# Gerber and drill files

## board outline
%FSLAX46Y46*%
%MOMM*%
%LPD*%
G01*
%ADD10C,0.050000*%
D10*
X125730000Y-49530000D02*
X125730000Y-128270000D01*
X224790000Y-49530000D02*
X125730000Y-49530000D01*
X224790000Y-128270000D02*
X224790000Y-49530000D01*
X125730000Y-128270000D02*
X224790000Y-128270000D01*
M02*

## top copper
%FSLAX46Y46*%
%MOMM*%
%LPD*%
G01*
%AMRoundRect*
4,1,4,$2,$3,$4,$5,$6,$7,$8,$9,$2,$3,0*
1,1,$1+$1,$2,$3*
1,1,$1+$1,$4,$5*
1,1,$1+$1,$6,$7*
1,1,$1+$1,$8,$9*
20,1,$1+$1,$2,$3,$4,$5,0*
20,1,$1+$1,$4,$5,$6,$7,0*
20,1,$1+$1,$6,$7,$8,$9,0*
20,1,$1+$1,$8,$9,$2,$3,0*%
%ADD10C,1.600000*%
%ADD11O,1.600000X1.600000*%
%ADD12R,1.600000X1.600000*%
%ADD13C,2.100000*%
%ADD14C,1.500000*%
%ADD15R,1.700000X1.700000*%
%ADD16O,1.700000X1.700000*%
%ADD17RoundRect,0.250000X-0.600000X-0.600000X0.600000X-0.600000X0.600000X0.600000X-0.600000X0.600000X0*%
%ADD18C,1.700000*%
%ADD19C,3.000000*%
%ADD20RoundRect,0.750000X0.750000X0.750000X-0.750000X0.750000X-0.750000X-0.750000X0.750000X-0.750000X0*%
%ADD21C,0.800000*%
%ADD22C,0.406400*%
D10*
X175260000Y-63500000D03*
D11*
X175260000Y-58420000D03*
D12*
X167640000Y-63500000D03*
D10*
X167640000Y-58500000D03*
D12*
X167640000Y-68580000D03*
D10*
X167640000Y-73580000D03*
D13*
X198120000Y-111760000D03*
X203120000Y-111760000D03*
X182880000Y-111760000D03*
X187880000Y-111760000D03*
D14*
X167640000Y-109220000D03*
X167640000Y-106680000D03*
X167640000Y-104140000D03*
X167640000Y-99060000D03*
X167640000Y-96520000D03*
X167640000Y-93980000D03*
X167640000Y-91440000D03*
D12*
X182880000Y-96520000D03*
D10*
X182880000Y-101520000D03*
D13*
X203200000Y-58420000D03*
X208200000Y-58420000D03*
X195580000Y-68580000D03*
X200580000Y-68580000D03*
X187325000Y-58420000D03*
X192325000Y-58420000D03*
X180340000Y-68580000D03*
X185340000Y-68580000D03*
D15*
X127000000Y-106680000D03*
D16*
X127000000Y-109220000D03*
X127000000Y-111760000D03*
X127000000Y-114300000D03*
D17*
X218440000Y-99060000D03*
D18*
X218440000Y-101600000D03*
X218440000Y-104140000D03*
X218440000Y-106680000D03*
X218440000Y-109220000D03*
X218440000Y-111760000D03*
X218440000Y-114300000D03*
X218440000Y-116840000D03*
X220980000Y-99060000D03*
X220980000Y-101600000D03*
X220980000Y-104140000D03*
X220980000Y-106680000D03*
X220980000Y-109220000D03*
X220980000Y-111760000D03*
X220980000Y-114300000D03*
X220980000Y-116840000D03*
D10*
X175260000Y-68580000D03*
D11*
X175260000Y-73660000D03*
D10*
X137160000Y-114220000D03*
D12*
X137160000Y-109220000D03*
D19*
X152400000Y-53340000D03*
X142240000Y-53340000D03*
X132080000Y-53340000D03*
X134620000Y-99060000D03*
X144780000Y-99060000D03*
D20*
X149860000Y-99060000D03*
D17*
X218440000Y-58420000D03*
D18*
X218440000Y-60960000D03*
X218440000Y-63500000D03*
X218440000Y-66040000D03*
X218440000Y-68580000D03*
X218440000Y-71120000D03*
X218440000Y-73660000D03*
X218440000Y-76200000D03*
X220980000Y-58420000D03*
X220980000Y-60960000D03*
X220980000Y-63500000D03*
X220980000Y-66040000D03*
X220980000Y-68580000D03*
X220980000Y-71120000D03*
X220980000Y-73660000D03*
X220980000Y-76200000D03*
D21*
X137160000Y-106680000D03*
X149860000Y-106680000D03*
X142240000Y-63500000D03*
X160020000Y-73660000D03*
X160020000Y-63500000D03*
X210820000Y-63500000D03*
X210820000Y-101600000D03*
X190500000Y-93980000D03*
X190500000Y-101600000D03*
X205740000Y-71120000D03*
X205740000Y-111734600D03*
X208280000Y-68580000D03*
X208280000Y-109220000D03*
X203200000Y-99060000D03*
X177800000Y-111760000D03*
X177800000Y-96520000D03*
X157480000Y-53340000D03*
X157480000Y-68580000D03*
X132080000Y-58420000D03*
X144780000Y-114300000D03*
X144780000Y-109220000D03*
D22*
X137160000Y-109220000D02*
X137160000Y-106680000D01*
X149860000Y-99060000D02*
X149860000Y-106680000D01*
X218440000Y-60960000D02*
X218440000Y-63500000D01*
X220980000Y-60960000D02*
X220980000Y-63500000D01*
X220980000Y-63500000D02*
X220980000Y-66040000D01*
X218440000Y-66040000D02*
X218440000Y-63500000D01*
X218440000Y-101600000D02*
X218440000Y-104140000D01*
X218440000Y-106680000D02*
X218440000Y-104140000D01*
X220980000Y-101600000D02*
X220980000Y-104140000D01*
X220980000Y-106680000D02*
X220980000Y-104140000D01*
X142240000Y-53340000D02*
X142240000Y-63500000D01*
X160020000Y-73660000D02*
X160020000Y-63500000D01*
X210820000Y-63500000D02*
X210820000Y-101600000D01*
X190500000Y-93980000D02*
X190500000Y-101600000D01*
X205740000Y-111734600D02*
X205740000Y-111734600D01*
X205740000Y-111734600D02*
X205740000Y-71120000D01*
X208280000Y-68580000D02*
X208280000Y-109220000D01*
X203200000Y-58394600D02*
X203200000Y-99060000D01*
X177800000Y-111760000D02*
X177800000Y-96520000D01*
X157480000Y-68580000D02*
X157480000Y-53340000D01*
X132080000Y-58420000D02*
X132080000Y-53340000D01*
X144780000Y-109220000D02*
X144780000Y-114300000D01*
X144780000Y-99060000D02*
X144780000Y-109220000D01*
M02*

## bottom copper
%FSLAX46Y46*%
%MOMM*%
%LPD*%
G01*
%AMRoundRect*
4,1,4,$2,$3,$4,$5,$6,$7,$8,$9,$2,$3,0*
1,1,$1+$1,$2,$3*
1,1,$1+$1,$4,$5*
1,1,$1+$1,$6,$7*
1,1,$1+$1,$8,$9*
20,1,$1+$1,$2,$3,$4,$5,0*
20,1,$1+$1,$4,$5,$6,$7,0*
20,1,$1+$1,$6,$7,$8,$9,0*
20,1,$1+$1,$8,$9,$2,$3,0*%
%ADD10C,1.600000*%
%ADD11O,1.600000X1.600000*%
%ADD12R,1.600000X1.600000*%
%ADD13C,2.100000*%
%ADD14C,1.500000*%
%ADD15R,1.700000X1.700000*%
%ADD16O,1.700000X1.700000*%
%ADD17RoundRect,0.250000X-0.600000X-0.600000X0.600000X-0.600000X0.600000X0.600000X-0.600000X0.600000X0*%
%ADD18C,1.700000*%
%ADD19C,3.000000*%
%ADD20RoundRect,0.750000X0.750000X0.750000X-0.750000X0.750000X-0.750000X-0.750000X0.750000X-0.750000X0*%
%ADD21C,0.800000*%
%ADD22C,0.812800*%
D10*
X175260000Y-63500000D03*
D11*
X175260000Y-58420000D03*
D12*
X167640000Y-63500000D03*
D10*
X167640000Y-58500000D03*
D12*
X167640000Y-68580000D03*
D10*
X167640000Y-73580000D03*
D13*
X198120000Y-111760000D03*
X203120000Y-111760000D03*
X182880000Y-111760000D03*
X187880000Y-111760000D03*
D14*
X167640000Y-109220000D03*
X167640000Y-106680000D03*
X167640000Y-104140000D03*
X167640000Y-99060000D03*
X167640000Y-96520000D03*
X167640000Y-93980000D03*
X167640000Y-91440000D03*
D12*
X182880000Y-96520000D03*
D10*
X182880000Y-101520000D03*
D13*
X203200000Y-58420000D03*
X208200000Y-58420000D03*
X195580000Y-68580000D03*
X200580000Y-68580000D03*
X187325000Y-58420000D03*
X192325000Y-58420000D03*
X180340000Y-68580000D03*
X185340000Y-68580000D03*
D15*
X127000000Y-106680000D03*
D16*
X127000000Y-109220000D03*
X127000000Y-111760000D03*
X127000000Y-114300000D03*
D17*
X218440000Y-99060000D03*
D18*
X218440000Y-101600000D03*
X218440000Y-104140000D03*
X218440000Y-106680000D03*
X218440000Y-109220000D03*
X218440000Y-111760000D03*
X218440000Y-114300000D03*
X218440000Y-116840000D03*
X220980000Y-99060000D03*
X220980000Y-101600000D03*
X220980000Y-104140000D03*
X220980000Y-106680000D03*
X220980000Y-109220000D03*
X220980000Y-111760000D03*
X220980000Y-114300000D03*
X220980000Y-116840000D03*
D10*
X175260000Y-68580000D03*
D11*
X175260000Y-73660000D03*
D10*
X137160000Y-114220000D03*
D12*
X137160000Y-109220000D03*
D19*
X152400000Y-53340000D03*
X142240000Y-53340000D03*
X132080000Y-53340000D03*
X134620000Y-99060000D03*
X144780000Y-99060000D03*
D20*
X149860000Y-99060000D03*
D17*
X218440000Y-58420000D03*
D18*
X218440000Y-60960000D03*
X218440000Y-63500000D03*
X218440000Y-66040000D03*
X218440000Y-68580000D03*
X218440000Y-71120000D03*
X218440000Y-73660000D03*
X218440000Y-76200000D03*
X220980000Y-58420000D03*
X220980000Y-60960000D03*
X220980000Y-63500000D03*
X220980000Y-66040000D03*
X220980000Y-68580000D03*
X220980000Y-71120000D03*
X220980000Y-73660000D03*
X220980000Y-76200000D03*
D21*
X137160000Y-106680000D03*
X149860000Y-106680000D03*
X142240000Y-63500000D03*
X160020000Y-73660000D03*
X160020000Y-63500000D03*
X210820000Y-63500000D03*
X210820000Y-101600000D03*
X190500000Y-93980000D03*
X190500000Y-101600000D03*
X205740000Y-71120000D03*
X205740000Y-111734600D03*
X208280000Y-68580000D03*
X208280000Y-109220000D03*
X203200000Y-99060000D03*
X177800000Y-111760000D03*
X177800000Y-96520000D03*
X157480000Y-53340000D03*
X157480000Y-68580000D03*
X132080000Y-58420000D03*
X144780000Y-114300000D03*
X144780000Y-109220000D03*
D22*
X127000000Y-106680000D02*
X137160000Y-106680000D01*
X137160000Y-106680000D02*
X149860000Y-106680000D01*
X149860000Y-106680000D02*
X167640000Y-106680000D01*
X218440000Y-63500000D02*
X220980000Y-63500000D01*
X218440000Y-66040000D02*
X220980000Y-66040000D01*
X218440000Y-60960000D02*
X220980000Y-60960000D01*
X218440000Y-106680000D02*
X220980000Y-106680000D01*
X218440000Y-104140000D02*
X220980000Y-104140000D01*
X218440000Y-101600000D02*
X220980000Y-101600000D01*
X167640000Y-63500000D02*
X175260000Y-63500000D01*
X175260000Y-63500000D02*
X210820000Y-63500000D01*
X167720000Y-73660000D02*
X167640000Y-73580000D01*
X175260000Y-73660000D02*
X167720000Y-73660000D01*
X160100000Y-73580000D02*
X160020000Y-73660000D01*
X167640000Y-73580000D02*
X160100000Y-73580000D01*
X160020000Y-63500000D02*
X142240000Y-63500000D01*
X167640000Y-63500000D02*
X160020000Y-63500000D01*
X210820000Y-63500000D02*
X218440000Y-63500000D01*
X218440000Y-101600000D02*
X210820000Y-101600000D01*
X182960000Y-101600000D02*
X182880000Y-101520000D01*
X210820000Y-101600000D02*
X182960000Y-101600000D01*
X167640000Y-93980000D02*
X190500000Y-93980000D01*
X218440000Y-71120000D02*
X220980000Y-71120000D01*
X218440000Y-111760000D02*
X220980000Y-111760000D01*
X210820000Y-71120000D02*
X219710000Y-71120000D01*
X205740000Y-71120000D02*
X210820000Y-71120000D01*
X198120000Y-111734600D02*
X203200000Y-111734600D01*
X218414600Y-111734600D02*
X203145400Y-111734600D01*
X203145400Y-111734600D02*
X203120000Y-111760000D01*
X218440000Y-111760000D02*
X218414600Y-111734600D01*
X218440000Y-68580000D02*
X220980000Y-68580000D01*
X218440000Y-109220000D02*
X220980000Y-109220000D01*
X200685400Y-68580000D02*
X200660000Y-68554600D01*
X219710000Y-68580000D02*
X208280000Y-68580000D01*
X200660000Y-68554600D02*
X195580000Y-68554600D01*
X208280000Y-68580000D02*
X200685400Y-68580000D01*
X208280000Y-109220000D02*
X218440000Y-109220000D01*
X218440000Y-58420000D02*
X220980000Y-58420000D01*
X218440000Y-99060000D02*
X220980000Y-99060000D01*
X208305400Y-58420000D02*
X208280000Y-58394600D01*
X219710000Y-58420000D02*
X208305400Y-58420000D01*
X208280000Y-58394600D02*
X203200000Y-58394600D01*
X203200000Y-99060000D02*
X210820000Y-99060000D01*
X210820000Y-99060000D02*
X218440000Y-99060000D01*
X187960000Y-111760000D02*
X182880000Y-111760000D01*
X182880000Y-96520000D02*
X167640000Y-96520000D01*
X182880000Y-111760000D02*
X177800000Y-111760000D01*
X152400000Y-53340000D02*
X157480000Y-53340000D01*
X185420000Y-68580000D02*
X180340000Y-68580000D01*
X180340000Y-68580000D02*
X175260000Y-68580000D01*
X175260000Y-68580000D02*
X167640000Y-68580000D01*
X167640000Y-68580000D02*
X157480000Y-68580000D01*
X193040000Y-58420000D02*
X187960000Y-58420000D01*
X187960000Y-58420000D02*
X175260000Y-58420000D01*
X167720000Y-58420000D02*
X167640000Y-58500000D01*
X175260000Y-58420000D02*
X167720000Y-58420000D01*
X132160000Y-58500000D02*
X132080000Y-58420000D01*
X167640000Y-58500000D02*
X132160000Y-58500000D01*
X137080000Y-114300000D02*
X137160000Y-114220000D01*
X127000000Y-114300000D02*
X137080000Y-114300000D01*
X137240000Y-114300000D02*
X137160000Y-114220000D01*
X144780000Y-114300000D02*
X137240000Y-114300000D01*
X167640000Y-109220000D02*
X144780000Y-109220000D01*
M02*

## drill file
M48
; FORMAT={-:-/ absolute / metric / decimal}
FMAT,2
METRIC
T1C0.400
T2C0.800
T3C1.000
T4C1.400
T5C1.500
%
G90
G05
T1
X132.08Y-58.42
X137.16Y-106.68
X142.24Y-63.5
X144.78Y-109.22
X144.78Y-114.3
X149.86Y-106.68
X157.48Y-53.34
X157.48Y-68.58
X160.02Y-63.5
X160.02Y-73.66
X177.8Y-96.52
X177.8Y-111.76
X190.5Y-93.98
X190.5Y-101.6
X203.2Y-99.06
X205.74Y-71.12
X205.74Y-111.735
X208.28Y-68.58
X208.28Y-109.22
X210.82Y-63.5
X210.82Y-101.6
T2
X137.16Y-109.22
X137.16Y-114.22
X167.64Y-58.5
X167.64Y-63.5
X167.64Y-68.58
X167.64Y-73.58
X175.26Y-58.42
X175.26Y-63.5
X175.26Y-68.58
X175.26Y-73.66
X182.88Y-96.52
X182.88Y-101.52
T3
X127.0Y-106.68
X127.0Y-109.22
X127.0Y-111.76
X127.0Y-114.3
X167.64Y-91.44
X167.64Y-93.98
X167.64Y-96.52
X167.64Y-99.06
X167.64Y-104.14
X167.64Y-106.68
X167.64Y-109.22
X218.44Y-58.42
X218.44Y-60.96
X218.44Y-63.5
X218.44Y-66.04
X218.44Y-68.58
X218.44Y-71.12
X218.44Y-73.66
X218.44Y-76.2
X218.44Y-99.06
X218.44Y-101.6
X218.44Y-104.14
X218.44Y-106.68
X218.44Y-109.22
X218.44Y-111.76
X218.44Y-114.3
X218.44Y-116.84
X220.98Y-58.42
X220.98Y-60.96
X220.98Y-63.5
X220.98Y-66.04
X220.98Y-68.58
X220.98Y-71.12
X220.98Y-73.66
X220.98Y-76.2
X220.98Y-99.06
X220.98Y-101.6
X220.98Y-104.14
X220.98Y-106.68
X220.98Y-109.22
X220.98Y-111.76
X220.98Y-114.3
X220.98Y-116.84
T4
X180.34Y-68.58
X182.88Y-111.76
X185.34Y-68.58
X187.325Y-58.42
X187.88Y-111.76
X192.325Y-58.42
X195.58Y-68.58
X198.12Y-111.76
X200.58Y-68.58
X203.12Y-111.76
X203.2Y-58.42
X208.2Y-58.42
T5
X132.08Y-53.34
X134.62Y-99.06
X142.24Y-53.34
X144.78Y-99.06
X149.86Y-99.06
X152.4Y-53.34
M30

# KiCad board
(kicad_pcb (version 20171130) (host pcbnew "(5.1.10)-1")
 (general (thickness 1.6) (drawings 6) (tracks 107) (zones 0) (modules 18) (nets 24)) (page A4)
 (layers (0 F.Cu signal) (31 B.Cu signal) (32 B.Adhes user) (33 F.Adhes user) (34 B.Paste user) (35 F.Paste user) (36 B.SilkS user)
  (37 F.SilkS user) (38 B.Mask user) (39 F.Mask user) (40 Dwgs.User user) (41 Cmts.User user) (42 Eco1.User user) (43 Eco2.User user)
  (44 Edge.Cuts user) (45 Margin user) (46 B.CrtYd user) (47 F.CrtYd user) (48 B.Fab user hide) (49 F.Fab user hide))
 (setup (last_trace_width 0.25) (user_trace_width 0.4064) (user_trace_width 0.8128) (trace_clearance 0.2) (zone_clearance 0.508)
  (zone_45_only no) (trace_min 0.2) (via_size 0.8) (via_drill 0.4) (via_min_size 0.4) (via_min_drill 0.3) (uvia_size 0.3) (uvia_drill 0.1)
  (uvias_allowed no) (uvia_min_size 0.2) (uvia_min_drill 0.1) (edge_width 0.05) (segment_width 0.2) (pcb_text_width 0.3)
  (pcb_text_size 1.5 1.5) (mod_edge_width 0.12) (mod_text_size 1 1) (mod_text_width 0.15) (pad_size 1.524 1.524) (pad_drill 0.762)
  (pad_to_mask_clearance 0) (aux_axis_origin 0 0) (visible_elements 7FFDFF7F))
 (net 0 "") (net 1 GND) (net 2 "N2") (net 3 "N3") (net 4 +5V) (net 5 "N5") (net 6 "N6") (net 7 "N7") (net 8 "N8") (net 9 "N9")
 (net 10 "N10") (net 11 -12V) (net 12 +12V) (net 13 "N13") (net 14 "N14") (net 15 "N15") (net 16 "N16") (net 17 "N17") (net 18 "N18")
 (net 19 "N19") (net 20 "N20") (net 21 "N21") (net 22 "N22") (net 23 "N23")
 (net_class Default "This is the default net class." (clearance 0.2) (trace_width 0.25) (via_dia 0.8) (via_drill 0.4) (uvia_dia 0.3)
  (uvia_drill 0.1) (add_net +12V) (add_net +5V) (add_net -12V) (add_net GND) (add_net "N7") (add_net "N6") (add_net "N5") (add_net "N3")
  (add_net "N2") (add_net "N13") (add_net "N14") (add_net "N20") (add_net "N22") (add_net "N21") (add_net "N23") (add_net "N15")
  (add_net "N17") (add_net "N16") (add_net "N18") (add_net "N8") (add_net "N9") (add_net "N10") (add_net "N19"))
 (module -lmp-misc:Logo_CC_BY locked (layer F.Cu) (at 163.449 124.333)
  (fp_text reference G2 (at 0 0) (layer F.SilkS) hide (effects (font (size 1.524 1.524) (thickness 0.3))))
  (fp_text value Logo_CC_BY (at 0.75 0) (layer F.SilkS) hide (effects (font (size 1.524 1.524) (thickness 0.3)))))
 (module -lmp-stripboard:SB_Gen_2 (layer F.Cu) (at 175.26 63.5 90)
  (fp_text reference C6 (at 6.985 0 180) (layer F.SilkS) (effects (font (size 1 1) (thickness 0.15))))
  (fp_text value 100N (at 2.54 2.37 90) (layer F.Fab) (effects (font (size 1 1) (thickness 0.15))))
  (pad 1 thru_hole circle (at 0 0 90) (size 1.6 1.6) (drill 0.8) (layers *.Cu *.Mask) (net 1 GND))
  (pad 2 thru_hole oval (at 5.08 0 90) (size 1.6 1.6) (drill 0.8) (layers *.Cu *.Mask) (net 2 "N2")))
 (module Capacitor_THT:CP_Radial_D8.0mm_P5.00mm (layer F.Cu) (at 167.64 63.5 90)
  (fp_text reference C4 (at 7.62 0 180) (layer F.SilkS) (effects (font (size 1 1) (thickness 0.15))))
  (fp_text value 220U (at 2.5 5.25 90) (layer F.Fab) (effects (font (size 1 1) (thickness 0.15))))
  (pad 1 thru_hole rect (at 0 0 90) (size 1.6 1.6) (drill 0.8) (layers *.Cu *.Mask) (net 1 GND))
  (pad 2 thru_hole circle (at 5 0 90) (size 1.6 1.6) (drill 0.8) (layers *.Cu *.Mask) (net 2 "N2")))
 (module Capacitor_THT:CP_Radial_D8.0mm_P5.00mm (layer F.Cu) (at 167.64 68.58 270)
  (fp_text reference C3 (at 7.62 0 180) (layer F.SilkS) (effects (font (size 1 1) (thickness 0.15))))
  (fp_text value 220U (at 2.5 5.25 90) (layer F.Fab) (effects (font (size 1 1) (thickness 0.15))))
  (pad 1 thru_hole rect (at 0 0 270) (size 1.6 1.6) (drill 0.8) (layers *.Cu *.Mask) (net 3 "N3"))
  (pad 2 thru_hole circle (at 5 0 270) (size 1.6 1.6) (drill 0.8) (layers *.Cu *.Mask) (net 1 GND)))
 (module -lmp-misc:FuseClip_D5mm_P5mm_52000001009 (layer F.Cu) (at 198.12 111.76)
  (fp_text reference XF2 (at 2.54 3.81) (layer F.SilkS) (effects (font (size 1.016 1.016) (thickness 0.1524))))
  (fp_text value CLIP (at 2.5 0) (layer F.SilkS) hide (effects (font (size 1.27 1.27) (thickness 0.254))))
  (pad 1 thru_hole circle (at 0 0) (size 2.1 2.1) (drill 1.4) (layers *.Cu *.Mask) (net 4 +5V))
  (pad 1 thru_hole circle (at 5 0) (size 2.1 2.1) (drill 1.4) (layers *.Cu *.Mask) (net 4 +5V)))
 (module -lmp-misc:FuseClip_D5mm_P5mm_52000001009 (layer F.Cu) (at 182.88 111.76)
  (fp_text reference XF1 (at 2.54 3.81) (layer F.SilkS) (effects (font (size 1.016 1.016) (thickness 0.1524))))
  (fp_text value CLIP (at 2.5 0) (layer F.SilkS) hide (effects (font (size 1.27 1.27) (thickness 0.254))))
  (pad 1 thru_hole circle (at 0 0) (size 2.1 2.1) (drill 1.4) (layers *.Cu *.Mask) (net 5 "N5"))
  (pad 1 thru_hole circle (at 5 0) (size 2.1 2.1) (drill 1.4) (layers *.Cu *.Mask) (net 5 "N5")))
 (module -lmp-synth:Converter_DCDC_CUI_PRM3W (layer F.Cu) (at 167.64 109.22 90)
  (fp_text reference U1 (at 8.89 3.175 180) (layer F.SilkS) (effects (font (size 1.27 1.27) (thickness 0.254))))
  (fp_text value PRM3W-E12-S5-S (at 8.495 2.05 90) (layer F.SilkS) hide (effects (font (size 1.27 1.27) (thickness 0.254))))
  (pad 1 thru_hole circle (at 0 0 90) (size 1.5 1.5) (drill 1) (layers *.Cu *.Mask) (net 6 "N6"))
  (pad 2 thru_hole circle (at 2.54 0 90) (size 1.5 1.5) (drill 1) (layers *.Cu *.Mask) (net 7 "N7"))
  (pad 3 thru_hole circle (at 5.08 0 90) (size 1.5 1.5) (drill 1) (layers *.Cu *.Mask) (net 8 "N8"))
  (pad 5 thru_hole circle (at 10.16 0 90) (size 1.5 1.5) (drill 1) (layers *.Cu *.Mask) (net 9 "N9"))
  (pad 6 thru_hole circle (at 12.7 0 90) (size 1.5 1.5) (drill 1) (layers *.Cu *.Mask) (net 5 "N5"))
  (pad 7 thru_hole circle (at 15.24 0 90) (size 1.5 1.5) (drill 1) (layers *.Cu *.Mask) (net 1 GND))
  (pad 8 thru_hole circle (at 17.78 0 90) (size 1.5 1.5) (drill 1) (layers *.Cu *.Mask) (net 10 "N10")))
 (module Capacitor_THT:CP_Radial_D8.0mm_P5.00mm (layer F.Cu) (at 182.88 96.52 270)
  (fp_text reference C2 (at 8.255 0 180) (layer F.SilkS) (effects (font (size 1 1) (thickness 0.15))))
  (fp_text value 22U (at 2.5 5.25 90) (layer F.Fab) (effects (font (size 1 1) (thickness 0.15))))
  (pad 1 thru_hole rect (at 0 0 270) (size 1.6 1.6) (drill 0.8) (layers *.Cu *.Mask) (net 5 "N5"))
  (pad 2 thru_hole circle (at 5 0 270) (size 1.6 1.6) (drill 0.8) (layers *.Cu *.Mask) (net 1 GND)))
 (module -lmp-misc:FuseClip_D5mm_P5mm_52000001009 (layer F.Cu) (at 203.2 58.42)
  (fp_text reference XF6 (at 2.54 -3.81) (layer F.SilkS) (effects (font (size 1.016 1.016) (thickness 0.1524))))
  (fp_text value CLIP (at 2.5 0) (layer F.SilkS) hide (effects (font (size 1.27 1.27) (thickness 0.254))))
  (pad 1 thru_hole circle (at 0 0) (size 2.1 2.1) (drill 1.4) (layers *.Cu *.Mask) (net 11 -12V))
  (pad 1 thru_hole circle (at 5 0) (size 2.1 2.1) (drill 1.4) (layers *.Cu *.Mask) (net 11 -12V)))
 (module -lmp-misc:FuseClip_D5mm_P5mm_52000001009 (layer F.Cu) (at 195.58 68.58)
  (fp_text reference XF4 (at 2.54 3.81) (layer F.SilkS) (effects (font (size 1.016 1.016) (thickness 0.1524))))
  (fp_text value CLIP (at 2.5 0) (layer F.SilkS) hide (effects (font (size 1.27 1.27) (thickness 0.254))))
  (pad 1 thru_hole circle (at 0 0) (size 2.1 2.1) (drill 1.4) (layers *.Cu *.Mask) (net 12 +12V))
  (pad 1 thru_hole circle (at 5 0) (size 2.1 2.1) (drill 1.4) (layers *.Cu *.Mask) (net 12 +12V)))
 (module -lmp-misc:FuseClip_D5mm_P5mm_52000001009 (layer F.Cu) (at 187.325 58.42)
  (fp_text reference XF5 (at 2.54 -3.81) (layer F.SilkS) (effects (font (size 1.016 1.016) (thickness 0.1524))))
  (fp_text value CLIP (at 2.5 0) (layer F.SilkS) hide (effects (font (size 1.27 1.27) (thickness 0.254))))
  (pad 1 thru_hole circle (at 0 0) (size 2.1 2.1) (drill 1.4) (layers *.Cu *.Mask) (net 2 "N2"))
  (pad 1 thru_hole circle (at 5 0) (size 2.1 2.1) (drill 1.4) (layers *.Cu *.Mask) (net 2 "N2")))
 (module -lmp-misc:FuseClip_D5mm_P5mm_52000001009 (layer F.Cu) (at 180.34 68.58)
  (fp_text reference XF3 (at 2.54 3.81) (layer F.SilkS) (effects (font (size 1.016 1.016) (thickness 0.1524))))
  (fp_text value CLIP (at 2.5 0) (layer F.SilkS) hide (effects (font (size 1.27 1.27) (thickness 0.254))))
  (pad 1 thru_hole circle (at 0 0) (size 2.1 2.1) (drill 1.4) (layers *.Cu *.Mask) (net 3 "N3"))
  (pad 1 thru_hole circle (at 5 0) (size 2.1 2.1) (drill 1.4) (layers *.Cu *.Mask) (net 3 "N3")))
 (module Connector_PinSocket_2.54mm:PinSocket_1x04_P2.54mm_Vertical (layer F.Cu) (at 127 106.68)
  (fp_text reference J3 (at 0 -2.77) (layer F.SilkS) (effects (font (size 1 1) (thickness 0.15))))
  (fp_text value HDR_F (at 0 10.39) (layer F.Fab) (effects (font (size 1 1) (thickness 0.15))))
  (pad 1 thru_hole rect (at 0 0) (size 1.7 1.7) (drill 1) (layers *.Cu *.Mask) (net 7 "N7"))
  (pad 2 thru_hole oval (at 0 2.54) (size 1.7 1.7) (drill 1) (layers *.Cu *.Mask) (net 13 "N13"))
  (pad 3 thru_hole oval (at 0 5.08) (size 1.7 1.7) (drill 1) (layers *.Cu *.Mask) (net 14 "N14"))
  (pad 4 thru_hole oval (at 0 7.62) (size 1.7 1.7) (drill 1) (layers *.Cu *.Mask) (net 6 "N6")))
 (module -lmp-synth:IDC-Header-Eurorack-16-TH (layer F.Cu) (at 218.44 99.06 180)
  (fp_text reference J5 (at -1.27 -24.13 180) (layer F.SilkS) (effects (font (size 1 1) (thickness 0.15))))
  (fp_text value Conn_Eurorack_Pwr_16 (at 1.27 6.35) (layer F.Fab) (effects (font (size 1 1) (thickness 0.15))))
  (pad 1 thru_hole roundrect (at 0 0) (size 1.7 1.7) (drill 1) (layers *.Cu *.Mask) (roundrect_rratio 0.147059) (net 11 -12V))
  (pad 3 thru_hole circle (at 0 -2.54) (size 1.7 1.7) (drill 1) (layers *.Cu *.Mask) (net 1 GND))
  (pad 5 thru_hole circle (at 0 -5.08) (size 1.7 1.7) (drill 1) (layers *.Cu *.Mask) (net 1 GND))
  (pad 7 thru_hole circle (at 0 -7.62) (size 1.7 1.7) (drill 1) (layers *.Cu *.Mask) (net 1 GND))
  (pad 9 thru_hole circle (at 0 -10.16) (size 1.7 1.7) (drill 1) (layers *.Cu *.Mask) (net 12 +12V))
  (pad 11 thru_hole circle (at 0 -12.7) (size 1.7 1.7) (drill 1) (layers *.Cu *.Mask) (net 4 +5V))
  (pad 13 thru_hole circle (at 0 -15.24) (size 1.7 1.7) (drill 1) (layers *.Cu *.Mask) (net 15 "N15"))
  (pad 15 thru_hole circle (at 0 -17.78) (size 1.7 1.7) (drill 1) (layers *.Cu *.Mask) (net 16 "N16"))
  (pad 2 thru_hole circle (at -2.54 0) (size 1.7 1.7) (drill 1) (layers *.Cu *.Mask) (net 11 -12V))
  (pad 4 thru_hole circle (at -2.54 -2.54) (size 1.7 1.7) (drill 1) (layers *.Cu *.Mask) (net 1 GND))
  (pad 6 thru_hole circle (at -2.54 -5.08) (size 1.7 1.7) (drill 1) (layers *.Cu *.Mask) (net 1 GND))
  (pad 8 thru_hole circle (at -2.54 -7.62) (size 1.7 1.7) (drill 1) (layers *.Cu *.Mask) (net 1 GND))
  (pad 10 thru_hole circle (at -2.54 -10.16) (size 1.7 1.7) (drill 1) (layers *.Cu *.Mask) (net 12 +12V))
  (pad 12 thru_hole circle (at -2.54 -12.7) (size 1.7 1.7) (drill 1) (layers *.Cu *.Mask) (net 4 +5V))
  (pad 14 thru_hole circle (at -2.54 -15.24) (size 1.7 1.7) (drill 1) (layers *.Cu *.Mask) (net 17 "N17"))
  (pad 16 thru_hole circle (at -2.54 -17.78) (size 1.7 1.7) (drill 1) (layers *.Cu *.Mask) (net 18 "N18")))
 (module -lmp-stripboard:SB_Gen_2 (layer F.Cu) (at 175.26 68.58 270)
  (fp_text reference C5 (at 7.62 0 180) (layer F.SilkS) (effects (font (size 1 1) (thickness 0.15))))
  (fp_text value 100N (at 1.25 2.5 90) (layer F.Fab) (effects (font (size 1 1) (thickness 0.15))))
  (pad 1 thru_hole circle (at 0 0 270) (size 1.6 1.6) (drill 0.8) (layers *.Cu *.Mask) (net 3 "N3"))
  (pad 2 thru_hole oval (at 5.08 0 270) (size 1.6 1.6) (drill 0.8) (layers *.Cu *.Mask) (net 1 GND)))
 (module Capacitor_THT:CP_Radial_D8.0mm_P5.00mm (layer F.Cu) (at 137.16 109.22 270)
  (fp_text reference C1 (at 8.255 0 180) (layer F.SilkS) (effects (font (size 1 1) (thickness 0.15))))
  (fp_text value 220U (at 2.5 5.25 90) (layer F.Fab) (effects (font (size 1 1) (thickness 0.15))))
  (pad 2 thru_hole circle (at 5 0 270) (size 1.6 1.6) (drill 0.8) (layers *.Cu *.Mask) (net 6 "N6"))
  (pad 1 thru_hole rect (at 0 0 270) (size 1.6 1.6) (drill 0.8) (layers *.Cu *.Mask) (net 7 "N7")))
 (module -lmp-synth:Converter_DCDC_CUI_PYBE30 (layer F.Cu) (at 149.86 99.06 180)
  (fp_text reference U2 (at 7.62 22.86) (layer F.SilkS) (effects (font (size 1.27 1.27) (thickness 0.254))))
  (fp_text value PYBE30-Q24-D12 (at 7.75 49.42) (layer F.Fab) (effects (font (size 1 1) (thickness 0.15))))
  (pad 6 thru_hole circle (at -2.54 45.72 180) (size 3 3) (drill 1.5) (layers *.Cu *.Mask) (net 3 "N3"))
  (pad 5 thru_hole circle (at 7.62 45.72 180) (size 3 3) (drill 1.5) (layers *.Cu *.Mask) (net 1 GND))
  (pad 4 thru_hole circle (at 17.78 45.72 180) (size 3 3) (drill 1.5) (layers *.Cu *.Mask) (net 2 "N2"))
  (pad 3 thru_hole circle (at 15.24 0 180) (size 3 3) (drill 1.5) (layers *.Cu *.Mask) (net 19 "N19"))
  (pad 2 thru_hole circle (at 5.08 0 180) (size 3 3) (drill 1.5) (layers *.Cu *.Mask) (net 6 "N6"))
  (pad 1 thru_hole roundrect (at 0 0 180) (size 3 3) (drill 1.5) (layers *.Cu *.Mask) (roundrect_rratio 0.25) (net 7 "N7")))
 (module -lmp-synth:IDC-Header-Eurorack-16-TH (layer F.Cu) (at 218.44 58.42 180)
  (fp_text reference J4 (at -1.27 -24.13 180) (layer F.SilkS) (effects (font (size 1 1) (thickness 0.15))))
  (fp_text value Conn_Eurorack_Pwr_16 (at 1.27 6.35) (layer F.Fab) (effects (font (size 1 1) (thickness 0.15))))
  (pad 1 thru_hole roundrect (at 0 0) (size 1.7 1.7) (drill 1) (layers *.Cu *.Mask) (roundrect_rratio 0.147059) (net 11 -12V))
  (pad 3 thru_hole circle (at 0 -2.54) (size 1.7 1.7) (drill 1) (layers *.Cu *.Mask) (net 1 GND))
  (pad 5 thru_hole circle (at 0 -5.08) (size 1.7 1.7) (drill 1) (layers *.Cu *.Mask) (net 1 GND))
  (pad 7 thru_hole circle (at 0 -7.62) (size 1.7 1.7) (drill 1) (layers *.Cu *.Mask) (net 1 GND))
  (pad 9 thru_hole circle (at 0 -10.16) (size 1.7 1.7) (drill 1) (layers *.Cu *.Mask) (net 12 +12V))
  (pad 11 thru_hole circle (at 0 -12.7) (size 1.7 1.7) (drill 1) (layers *.Cu *.Mask) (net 4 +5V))
  (pad 13 thru_hole circle (at 0 -15.24) (size 1.7 1.7) (drill 1) (layers *.Cu *.Mask) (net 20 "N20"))
  (pad 15 thru_hole circle (at 0 -17.78) (size 1.7 1.7) (drill 1) (layers *.Cu *.Mask) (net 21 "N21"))
  (pad 2 thru_hole circle (at -2.54 0) (size 1.7 1.7) (drill 1) (layers *.Cu *.Mask) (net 11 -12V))
  (pad 4 thru_hole circle (at -2.54 -2.54) (size 1.7 1.7) (drill 1) (layers *.Cu *.Mask) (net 1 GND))
  (pad 6 thru_hole circle (at -2.54 -5.08) (size 1.7 1.7) (drill 1) (layers *.Cu *.Mask) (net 1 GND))
  (pad 8 thru_hole circle (at -2.54 -7.62) (size 1.7 1.7) (drill 1) (layers *.Cu *.Mask) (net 1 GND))
  (pad 10 thru_hole circle (at -2.54 -10.16) (size 1.7 1.7) (drill 1) (layers *.Cu *.Mask) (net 12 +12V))
  (pad 12 thru_hole circle (at -2.54 -12.7) (size 1.7 1.7) (drill 1) (layers *.Cu *.Mask) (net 4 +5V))
  (pad 14 thru_hole circle (at -2.54 -15.24) (size 1.7 1.7) (drill 1) (layers *.Cu *.Mask) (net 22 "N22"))
  (pad 16 thru_hole circle (at -2.54 -17.78) (size 1.7 1.7) (drill 1) (layers *.Cu *.Mask) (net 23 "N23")))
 (gr_line (start 125.73 49.53) (end 125.73 128.27) (layer Edge.Cuts) (width 0.05))
 (gr_line (start 224.79 49.53) (end 125.73 49.53) (layer Edge.Cuts) (width 0.05))
 (gr_line (start 224.79 128.27) (end 224.79 49.53) (layer Edge.Cuts) (width 0.05))
 (gr_line (start 125.73 128.27) (end 224.79 128.27) (layer Edge.Cuts) (width 0.05))
 (via (at 137.16 106.68) (size 0.8) (drill 0.4) (layers F.Cu B.Cu) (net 7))
 (segment (start 137.16 109.22) (end 137.16 106.68) (width 0.4064) (layer F.Cu) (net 7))
 (segment (start 127 106.68) (end 137.16 106.68) (width 0.8128) (layer B.Cu) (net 7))
 (via (at 149.86 106.68) (size 0.8) (drill 0.4) (layers F.Cu B.Cu) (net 7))
 (segment (start 149.86 99.06) (end 149.86 106.68) (width 0.4064) (layer F.Cu) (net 7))
 (segment (start 137.16 106.68) (end 149.86 106.68) (width 0.8128) (layer B.Cu) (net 7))
 (segment (start 149.86 106.68) (end 167.64 106.68) (width 0.8128) (layer B.Cu) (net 7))
 (segment (start 218.44 63.5) (end 220.98 63.5) (width 0.8128) (layer B.Cu) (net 1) (status 30))
 (segment (start 218.44 66.04) (end 220.98 66.04) (width 0.8128) (layer B.Cu) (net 1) (status 30))
 (segment (start 218.44 60.96) (end 220.98 60.96) (width 0.8128) (layer B.Cu) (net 1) (status 30))
 (segment (start 218.44 60.96) (end 218.44 63.5) (width 0.4064) (layer F.Cu) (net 1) (status 30))
 (segment (start 220.98 60.96) (end 220.98 63.5) (width 0.4064) (layer F.Cu) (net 1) (status 30))
 (segment (start 220.98 63.5) (end 220.98 66.04) (width 0.4064) (layer F.Cu) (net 1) (status 30))
 (segment (start 218.44 66.04) (end 218.44 63.5) (width 0.4064) (layer F.Cu) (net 1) (status 30))
 (segment (start 218.44 106.68) (end 220.98 106.68) (width 0.8128) (layer B.Cu) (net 1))
 (segment (start 218.44 104.14) (end 220.98 104.14) (width 0.8128) (layer B.Cu) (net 1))
 (segment (start 218.44 101.6) (end 220.98 101.6) (width 0.8128) (layer B.Cu) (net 1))
 (segment (start 218.44 101.6) (end 218.44 104.14) (width 0.4064) (layer F.Cu) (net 1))
 (segment (start 218.44 106.68) (end 218.44 104.14) (width 0.4064) (layer F.Cu) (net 1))
 (segment (start 220.98 101.6) (end 220.98 104.14) (width 0.4064) (layer F.Cu) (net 1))
 (segment (start 220.98 106.68) (end 220.98 104.14) (width 0.4064) (layer F.Cu) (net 1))
 (segment (start 167.64 63.5) (end 175.26 63.5) (width 0.8128) (layer B.Cu) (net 1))
 (segment (start 175.26 63.5) (end 210.82 63.5) (width 0.8128) (layer B.Cu) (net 1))
 (via (at 142.24 63.5) (size 0.8) (drill 0.4) (layers F.Cu B.Cu) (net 1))
 (segment (start 142.24 53.34) (end 142.24 63.5) (width 0.4064) (layer F.Cu) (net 1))
 (segment (start 167.72 73.66) (end 167.64 73.58) (width 0.8128) (layer B.Cu) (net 1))
 (segment (start 175.26 73.66) (end 167.72 73.66) (width 0.8128) (layer B.Cu) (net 1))
 (via (at 160.02 73.66) (size 0.8) (drill 0.4) (layers F.Cu B.Cu) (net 1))
 (segment (start 160.1 73.58) (end 160.02 73.66) (width 0.8128) (layer B.Cu) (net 1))
 (segment (start 167.64 73.58) (end 160.1 73.58) (width 0.8128) (layer B.Cu) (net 1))
 (via (at 160.02 63.5) (size 0.8) (drill 0.4) (layers F.Cu B.Cu) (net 1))
 (segment (start 160.02 63.5) (end 142.24 63.5) (width 0.8128) (layer B.Cu) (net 1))
 (segment (start 160.02 73.66) (end 160.02 63.5) (width 0.4064) (layer F.Cu) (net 1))
 (segment (start 167.64 63.5) (end 160.02 63.5) (width 0.8128) (layer B.Cu) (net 1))
 (segment (start 210.82 63.5) (end 218.44 63.5) (width 0.8128) (layer B.Cu) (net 1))
 (via (at 210.82 63.5) (size 0.8) (drill 0.4) (layers F.Cu B.Cu) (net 1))
 (segment (start 218.44 101.6) (end 210.82 101.6) (width 0.8128) (layer B.Cu) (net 1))
 (via (at 210.82 101.6) (size 0.8) (drill 0.4) (layers F.Cu B.Cu) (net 1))
 (segment (start 210.82 63.5) (end 210.82 101.6) (width 0.4064) (layer F.Cu) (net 1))
 (segment (start 182.96 101.6) (end 182.88 101.52) (width 0.8128) (layer B.Cu) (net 1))
 (segment (start 210.82 101.6) (end 182.96 101.6) (width 0.8128) (layer B.Cu) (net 1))
 (via (at 190.5 93.98) (size 0.8) (drill 0.4) (layers F.Cu B.Cu) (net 1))
 (segment (start 167.64 93.98) (end 190.5 93.98) (width 0.8128) (layer B.Cu) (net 1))
 (segment (start 190.5 93.98) (end 190.5 101.6) (width 0.4064) (layer F.Cu) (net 1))
 (via (at 190.5 101.6) (size 0.8) (drill 0.4) (layers F.Cu B.Cu) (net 1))
 (segment (start 218.44 71.12) (end 220.98 71.12) (width 0.8128) (layer B.Cu) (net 4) (status 30))
 (segment (start 218.44 111.76) (end 220.98 111.76) (width 0.8128) (layer B.Cu) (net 4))
 (via (at 205.74 71.12) (size 0.8) (drill 0.4) (layers F.Cu B.Cu) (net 4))
 (segment (start 210.82 71.12) (end 219.71 71.12) (width 0.8128) (layer B.Cu) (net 4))
 (segment (start 205.74 71.12) (end 210.82 71.12) (width 0.8128) (layer B.Cu) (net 4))
 (segment (start 198.12 111.7346) (end 203.2 111.7346) (width 0.8128) (layer B.Cu) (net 4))
 (segment (start 205.74 111.7346) (end 205.74 111.7346) (width 0.4064) (layer F.Cu) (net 4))
 (segment (start 218.4146 111.7346) (end 203.1454 111.7346) (width 0.8128) (layer B.Cu) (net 4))
 (segment (start 203.1454 111.7346) (end 203.12 111.76) (width 0.8128) (layer B.Cu) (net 4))
 (segment (start 218.44 111.76) (end 218.4146 111.7346) (width 0.8128) (layer B.Cu) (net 4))
 (segment (start 205.74 111.7346) (end 205.74 71.12) (width 0.4064) (layer F.Cu) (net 4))
 (via (at 205.74 111.7346) (size 0.8) (drill 0.4) (layers F.Cu B.Cu) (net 4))
 (segment (start 218.44 68.58) (end 220.98 68.58) (width 0.8128) (layer B.Cu) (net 12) (status 30))
 (segment (start 218.44 109.22) (end 220.98 109.22) (width 0.8128) (layer B.Cu) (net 12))
 (segment (start 200.6854 68.58) (end 200.66 68.5546) (width 0.8128) (layer B.Cu) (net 12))
 (segment (start 219.71 68.58) (end 208.28 68.58) (width 0.8128) (layer B.Cu) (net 12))
 (segment (start 200.66 68.5546) (end 195.58 68.5546) (width 0.8128) (layer B.Cu) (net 12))
 (segment (start 208.28 68.58) (end 200.6854 68.58) (width 0.8128) (layer B.Cu) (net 12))
 (via (at 208.28 68.58) (size 0.8) (drill 0.4) (layers F.Cu B.Cu) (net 12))
 (segment (start 208.28 68.58) (end 208.28 109.22) (width 0.4064) (layer F.Cu) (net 12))
 (via (at 208.28 109.22) (size 0.8) (drill 0.4) (layers F.Cu B.Cu) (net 12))
 (segment (start 208.28 109.22) (end 218.44 109.22) (width 0.8128) (layer B.Cu) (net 12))
 (segment (start 218.44 58.42) (end 220.98 58.42) (width 0.8128) (layer B.Cu) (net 11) (status 30))
 (segment (start 218.44 99.06) (end 220.98 99.06) (width 0.8128) (layer B.Cu) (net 11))
 (segment (start 208.3054 58.42) (end 208.28 58.3946) (width 0.8128) (layer B.Cu) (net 11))
 (segment (start 219.71 58.42) (end 208.3054 58.42) (width 0.8128) (layer B.Cu) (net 11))
 (segment (start 208.28 58.3946) (end 203.2 58.3946) (width 0.8128) (layer B.Cu) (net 11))
 (segment (start 203.2 99.06) (end 210.82 99.06) (width 0.8128) (layer B.Cu) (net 11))
 (segment (start 210.82 99.06) (end 218.44 99.06) (width 0.8128) (layer B.Cu) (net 11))
 (via (at 203.2 99.06) (size 0.8) (drill 0.4) (layers F.Cu B.Cu) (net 11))
 (segment (start 203.2 58.3946) (end 203.2 99.06) (width 0.4064) (layer F.Cu) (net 11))
 (segment (start 187.96 111.76) (end 182.88 111.76) (width 0.8128) (layer B.Cu) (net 5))
 (segment (start 182.88 96.52) (end 167.64 96.52) (width 0.8128) (layer B.Cu) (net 5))
 (via (at 177.8 111.76) (size 0.8) (drill 0.4) (layers F.Cu B.Cu) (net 5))
 (segment (start 182.88 111.76) (end 177.8 111.76) (width 0.8128) (layer B.Cu) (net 5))
 (segment (start 177.8 111.76) (end 177.8 96.52) (width 0.4064) (layer F.Cu) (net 5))
 (via (at 177.8 96.52) (size 0.8) (drill 0.4) (layers F.Cu B.Cu) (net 5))
 (via (at 157.48 53.34) (size 0.8) (drill 0.4) (layers F.Cu B.Cu) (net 3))
 (segment (start 152.4 53.34) (end 157.48 53.34) (width 0.8128) (layer B.Cu) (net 3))
 (segment (start 185.42 68.58) (end 180.34 68.58) (width 0.8128) (layer B.Cu) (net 3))
 (segment (start 180.34 68.58) (end 175.26 68.58) (width 0.8128) (layer B.Cu) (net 3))
 (segment (start 175.26 68.58) (end 167.64 68.58) (width 0.8128) (layer B.Cu) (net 3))
 (via (at 157.48 68.58) (size 0.8) (drill 0.4) (layers F.Cu B.Cu) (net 3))
 (segment (start 167.64 68.58) (end 157.48 68.58) (width 0.8128) (layer B.Cu) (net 3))
 (segment (start 157.48 68.58) (end 157.48 53.34) (width 0.4064) (layer F.Cu) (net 3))
 (segment (start 193.04 58.42) (end 187.96 58.42) (width 0.8128) (layer B.Cu) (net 2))
 (segment (start 187.96 58.42) (end 175.26 58.42) (width 0.8128) (layer B.Cu) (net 2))
 (segment (start 167.72 58.42) (end 167.64 58.5) (width 0.8128) (layer B.Cu) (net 2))
 (segment (start 175.26 58.42) (end 167.72 58.42) (width 0.8128) (layer B.Cu) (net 2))
 (via (at 132.08 58.42) (size 0.8) (drill 0.4) (layers F.Cu B.Cu) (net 2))
 (segment (start 132.16 58.5) (end 132.08 58.42) (width 0.8128) (layer B.Cu) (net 2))
 (segment (start 167.64 58.5) (end 132.16 58.5) (width 0.8128) (layer B.Cu) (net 2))
 (segment (start 132.08 58.42) (end 132.08 53.34) (width 0.4064) (layer F.Cu) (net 2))
 (segment (start 137.08 114.3) (end 137.16 114.22) (width 0.8128) (layer B.Cu) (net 6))
 (segment (start 127 114.3) (end 137.08 114.3) (width 0.8128) (layer B.Cu) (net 6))
 (via (at 144.78 114.3) (size 0.8) (drill 0.4) (layers F.Cu B.Cu) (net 6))
 (segment (start 137.24 114.3) (end 137.16 114.22) (width 0.8128) (layer B.Cu) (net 6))
 (segment (start 144.78 114.3) (end 137.24 114.3) (width 0.8128) (layer B.Cu) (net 6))
 (segment (start 144.78 109.22) (end 144.78 114.3) (width 0.4064) (layer F.Cu) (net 6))
 (segment (start 144.78 99.06) (end 144.78 109.22) (width 0.4064) (layer F.Cu) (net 6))
 (via (at 144.78 109.22) (size 0.8) (drill 0.4) (layers F.Cu B.Cu) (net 6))
 (segment (start 167.64 109.22) (end 144.78 109.22) (width 0.8128) (layer B.Cu) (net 6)))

